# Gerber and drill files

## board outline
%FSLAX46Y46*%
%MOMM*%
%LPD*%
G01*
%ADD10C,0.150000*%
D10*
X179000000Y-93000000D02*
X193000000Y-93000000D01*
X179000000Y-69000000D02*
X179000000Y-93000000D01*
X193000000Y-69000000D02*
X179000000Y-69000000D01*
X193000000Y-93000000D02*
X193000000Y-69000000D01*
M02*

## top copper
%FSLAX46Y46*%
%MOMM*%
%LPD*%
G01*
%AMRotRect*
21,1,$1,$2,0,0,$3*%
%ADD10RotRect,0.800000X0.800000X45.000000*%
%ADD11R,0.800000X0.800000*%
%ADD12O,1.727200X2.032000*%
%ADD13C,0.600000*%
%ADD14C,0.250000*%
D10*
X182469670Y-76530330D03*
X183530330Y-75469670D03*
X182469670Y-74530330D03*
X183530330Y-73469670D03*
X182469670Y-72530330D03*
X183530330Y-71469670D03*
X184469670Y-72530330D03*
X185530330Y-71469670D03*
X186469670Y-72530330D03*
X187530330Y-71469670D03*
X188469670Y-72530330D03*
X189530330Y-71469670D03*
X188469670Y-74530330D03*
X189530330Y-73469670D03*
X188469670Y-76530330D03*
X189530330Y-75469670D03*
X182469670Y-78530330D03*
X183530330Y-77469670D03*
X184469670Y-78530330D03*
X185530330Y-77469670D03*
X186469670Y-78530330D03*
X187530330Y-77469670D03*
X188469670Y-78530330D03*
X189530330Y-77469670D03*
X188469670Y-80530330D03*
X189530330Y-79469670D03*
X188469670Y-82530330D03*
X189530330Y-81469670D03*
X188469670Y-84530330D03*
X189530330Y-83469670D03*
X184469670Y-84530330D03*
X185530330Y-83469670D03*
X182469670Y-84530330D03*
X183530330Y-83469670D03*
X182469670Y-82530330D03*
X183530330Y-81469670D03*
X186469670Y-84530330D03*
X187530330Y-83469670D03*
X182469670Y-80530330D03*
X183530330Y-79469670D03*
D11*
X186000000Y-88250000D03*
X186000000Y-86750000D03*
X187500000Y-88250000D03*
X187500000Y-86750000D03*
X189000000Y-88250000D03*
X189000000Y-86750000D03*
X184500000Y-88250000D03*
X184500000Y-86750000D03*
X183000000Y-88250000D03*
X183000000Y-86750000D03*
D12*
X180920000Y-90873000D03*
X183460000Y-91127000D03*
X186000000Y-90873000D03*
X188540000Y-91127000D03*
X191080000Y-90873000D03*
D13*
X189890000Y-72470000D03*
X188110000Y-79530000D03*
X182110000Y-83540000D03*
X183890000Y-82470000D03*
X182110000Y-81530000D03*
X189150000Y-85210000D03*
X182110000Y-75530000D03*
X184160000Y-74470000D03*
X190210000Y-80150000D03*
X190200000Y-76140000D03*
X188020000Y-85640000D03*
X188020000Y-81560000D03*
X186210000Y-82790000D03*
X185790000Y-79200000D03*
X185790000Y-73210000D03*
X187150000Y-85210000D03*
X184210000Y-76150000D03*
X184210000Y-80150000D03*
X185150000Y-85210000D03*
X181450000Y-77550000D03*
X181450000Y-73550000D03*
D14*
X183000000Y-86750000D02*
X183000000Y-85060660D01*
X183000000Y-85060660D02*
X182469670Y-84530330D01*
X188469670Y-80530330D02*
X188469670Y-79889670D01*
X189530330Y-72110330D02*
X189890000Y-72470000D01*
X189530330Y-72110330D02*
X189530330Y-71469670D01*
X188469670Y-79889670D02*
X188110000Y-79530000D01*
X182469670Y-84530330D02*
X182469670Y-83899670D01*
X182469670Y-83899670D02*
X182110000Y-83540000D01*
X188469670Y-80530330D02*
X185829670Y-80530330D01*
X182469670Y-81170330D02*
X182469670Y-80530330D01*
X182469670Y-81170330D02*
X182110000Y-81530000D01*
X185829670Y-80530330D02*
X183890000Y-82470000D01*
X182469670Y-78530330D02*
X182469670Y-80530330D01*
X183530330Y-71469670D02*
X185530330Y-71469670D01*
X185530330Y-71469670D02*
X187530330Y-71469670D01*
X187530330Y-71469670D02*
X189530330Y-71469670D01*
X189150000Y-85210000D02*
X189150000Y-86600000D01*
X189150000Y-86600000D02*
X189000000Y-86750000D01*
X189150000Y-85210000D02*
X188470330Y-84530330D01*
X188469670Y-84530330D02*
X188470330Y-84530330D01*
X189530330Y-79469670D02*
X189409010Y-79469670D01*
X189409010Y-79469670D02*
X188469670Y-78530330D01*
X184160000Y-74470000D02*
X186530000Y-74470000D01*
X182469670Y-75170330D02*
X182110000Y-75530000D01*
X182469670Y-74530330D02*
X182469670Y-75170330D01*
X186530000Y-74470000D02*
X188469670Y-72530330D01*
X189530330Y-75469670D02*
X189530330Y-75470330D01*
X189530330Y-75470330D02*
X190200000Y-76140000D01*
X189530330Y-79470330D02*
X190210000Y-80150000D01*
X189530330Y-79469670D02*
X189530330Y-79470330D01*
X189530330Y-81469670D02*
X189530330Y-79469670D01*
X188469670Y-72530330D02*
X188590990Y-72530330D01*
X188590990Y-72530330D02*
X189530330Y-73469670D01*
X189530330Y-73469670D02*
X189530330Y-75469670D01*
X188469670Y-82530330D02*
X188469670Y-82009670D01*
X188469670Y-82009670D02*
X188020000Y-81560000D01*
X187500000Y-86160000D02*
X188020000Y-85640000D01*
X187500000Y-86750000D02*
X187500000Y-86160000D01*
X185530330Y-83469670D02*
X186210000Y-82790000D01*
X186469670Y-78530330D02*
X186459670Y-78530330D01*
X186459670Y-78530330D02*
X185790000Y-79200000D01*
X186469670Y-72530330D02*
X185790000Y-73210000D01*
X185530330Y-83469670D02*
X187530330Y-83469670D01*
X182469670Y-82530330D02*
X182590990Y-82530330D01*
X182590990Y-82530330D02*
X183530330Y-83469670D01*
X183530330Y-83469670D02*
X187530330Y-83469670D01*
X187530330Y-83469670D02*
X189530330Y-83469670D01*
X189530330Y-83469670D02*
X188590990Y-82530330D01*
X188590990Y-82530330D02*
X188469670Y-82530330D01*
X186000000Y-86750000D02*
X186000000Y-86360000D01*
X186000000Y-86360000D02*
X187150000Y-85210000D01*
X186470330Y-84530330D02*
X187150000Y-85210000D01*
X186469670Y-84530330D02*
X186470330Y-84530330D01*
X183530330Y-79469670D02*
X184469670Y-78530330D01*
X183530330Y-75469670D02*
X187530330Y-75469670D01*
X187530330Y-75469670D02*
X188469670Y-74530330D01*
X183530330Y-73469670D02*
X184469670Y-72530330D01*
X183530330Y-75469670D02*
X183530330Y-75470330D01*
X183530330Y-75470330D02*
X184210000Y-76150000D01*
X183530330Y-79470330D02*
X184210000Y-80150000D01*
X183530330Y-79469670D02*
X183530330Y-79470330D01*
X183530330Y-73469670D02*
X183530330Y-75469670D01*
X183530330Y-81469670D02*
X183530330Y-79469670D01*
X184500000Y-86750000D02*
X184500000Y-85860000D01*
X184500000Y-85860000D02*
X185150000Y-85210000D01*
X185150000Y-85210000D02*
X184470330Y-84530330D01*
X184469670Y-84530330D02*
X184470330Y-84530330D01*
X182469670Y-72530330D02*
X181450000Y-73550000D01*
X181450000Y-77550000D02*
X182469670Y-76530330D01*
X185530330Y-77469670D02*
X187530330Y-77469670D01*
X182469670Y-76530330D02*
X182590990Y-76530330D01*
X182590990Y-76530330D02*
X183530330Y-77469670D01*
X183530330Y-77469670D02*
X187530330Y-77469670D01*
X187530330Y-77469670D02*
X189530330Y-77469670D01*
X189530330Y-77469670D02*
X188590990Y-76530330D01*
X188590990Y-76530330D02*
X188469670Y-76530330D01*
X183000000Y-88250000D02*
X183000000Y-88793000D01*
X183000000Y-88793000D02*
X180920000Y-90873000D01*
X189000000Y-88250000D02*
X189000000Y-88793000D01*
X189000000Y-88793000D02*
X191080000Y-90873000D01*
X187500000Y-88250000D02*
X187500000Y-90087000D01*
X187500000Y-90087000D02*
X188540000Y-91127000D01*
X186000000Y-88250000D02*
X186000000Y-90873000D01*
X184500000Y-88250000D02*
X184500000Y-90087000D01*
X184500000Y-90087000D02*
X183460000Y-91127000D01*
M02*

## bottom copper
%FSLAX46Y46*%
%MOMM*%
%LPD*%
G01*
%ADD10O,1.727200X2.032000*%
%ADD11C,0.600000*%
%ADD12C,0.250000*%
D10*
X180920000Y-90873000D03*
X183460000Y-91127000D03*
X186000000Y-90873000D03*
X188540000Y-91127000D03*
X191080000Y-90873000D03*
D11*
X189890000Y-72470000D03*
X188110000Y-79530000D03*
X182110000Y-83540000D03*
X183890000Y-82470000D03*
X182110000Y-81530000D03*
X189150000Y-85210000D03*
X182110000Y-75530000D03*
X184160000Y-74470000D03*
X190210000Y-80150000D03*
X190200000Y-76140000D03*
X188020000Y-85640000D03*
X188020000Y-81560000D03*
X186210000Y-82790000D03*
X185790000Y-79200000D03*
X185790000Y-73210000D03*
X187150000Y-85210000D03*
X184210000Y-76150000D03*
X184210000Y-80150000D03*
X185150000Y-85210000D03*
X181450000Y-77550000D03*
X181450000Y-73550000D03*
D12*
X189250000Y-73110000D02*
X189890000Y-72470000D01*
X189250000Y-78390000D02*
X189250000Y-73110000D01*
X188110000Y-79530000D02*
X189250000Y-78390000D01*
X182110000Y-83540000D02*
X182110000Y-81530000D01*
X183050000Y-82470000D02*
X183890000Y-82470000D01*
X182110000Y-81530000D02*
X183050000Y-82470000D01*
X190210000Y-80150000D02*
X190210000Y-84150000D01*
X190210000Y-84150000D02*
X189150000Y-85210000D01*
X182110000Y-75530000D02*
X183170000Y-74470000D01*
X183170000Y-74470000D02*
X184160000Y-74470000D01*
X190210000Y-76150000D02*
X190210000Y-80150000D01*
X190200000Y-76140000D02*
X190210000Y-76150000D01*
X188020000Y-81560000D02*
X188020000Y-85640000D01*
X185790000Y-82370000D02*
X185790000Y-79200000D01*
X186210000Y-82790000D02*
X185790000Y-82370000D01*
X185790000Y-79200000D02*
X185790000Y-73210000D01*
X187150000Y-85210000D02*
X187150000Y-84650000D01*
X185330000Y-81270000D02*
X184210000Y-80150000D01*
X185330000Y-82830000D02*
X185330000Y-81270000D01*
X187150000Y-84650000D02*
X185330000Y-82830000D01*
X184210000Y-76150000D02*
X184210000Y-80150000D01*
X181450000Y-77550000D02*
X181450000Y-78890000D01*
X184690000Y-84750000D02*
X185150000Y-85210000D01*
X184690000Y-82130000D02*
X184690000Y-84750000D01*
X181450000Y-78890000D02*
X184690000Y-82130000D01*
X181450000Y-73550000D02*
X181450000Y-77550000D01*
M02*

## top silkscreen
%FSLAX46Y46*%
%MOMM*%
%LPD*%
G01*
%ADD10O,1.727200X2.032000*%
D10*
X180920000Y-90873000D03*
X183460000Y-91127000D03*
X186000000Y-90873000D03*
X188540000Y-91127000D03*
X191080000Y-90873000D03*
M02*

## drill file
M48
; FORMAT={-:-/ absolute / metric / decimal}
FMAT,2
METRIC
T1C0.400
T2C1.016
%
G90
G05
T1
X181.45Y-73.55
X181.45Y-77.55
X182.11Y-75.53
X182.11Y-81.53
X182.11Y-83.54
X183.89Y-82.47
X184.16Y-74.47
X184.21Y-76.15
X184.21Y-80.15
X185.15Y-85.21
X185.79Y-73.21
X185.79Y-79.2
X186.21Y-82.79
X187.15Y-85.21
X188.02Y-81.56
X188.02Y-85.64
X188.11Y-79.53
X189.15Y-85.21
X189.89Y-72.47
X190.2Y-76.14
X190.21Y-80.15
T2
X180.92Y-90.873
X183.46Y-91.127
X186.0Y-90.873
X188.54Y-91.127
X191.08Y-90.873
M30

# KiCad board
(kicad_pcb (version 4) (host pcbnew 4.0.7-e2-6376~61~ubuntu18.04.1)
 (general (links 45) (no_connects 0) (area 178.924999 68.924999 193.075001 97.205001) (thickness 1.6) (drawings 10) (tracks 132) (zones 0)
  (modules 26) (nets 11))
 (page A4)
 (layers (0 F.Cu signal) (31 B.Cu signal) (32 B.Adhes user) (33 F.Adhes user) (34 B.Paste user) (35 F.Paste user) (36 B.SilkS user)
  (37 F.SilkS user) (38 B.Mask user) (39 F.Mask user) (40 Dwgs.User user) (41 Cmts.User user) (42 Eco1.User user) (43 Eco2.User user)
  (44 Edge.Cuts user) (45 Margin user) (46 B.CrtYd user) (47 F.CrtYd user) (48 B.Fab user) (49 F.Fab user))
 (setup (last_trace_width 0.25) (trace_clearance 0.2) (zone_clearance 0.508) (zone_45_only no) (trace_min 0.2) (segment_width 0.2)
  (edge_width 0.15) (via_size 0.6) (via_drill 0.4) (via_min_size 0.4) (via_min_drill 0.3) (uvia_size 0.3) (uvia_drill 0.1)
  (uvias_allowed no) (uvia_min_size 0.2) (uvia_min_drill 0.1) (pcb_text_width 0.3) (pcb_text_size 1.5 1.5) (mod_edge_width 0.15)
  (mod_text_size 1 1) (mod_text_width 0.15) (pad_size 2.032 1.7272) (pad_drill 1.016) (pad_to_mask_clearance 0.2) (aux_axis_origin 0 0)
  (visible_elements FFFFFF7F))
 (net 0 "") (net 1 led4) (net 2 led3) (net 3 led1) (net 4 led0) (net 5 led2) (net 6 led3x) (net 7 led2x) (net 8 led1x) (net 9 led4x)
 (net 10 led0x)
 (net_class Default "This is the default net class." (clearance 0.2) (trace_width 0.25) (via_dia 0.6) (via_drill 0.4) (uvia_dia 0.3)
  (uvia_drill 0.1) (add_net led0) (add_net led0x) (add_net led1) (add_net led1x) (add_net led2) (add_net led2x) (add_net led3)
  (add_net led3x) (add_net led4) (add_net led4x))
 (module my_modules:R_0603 (layer F.Cu) (at 183 76 45)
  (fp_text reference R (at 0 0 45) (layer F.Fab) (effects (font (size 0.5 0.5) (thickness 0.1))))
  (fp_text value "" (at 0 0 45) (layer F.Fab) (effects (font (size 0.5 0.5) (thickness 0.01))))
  (pad 1 smd rect (at -0.75 0 45) (size 0.8 0.8) (layers F.Cu F.Paste F.Mask) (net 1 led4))
  (pad 2 smd rect (at 0.75 0 45) (size 0.8 0.8) (layers F.Cu F.Paste F.Mask) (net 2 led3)))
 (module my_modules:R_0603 (layer F.Cu) (at 183 74 45)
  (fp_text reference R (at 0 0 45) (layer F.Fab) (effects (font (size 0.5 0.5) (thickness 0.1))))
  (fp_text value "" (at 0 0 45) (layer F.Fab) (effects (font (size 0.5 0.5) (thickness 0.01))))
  (pad 1 smd rect (at -0.75 0 45) (size 0.8 0.8) (layers F.Cu F.Paste F.Mask) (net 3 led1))
  (pad 2 smd rect (at 0.75 0 45) (size 0.8 0.8) (layers F.Cu F.Paste F.Mask) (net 2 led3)))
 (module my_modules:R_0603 (layer F.Cu) (at 183 72 45)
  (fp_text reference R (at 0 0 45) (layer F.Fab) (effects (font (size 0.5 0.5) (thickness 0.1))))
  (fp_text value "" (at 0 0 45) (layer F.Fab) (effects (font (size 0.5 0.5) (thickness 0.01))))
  (pad 1 smd rect (at -0.75 0 45) (size 0.8 0.8) (layers F.Cu F.Paste F.Mask) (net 1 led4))
  (pad 2 smd rect (at 0.75 0 45) (size 0.8 0.8) (layers F.Cu F.Paste F.Mask) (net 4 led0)))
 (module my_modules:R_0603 (layer F.Cu) (at 185 72 45)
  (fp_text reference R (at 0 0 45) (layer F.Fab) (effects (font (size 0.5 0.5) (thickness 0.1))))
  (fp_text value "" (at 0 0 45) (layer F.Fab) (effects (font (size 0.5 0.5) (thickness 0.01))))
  (pad 1 smd rect (at -0.75 0 45) (size 0.8 0.8) (layers F.Cu F.Paste F.Mask) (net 2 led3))
  (pad 2 smd rect (at 0.75 0 45) (size 0.8 0.8) (layers F.Cu F.Paste F.Mask) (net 4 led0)))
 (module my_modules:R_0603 (layer F.Cu) (at 187 72 45)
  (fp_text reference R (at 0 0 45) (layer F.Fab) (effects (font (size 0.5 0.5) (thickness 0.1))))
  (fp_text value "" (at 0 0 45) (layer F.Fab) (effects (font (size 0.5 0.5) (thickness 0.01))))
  (pad 1 smd rect (at -0.75 0 45) (size 0.8 0.8) (layers F.Cu F.Paste F.Mask) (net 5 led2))
  (pad 2 smd rect (at 0.75 0 45) (size 0.8 0.8) (layers F.Cu F.Paste F.Mask) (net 4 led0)))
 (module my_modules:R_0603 (layer F.Cu) (at 189 72 45)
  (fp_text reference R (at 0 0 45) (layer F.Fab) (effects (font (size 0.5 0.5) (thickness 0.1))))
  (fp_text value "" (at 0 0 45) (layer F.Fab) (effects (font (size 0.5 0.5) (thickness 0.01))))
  (pad 1 smd rect (at -0.75 0 45) (size 0.8 0.8) (layers F.Cu F.Paste F.Mask) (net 3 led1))
  (pad 2 smd rect (at 0.75 0 45) (size 0.8 0.8) (layers F.Cu F.Paste F.Mask) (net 4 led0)))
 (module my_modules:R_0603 (layer F.Cu) (at 189 74 45)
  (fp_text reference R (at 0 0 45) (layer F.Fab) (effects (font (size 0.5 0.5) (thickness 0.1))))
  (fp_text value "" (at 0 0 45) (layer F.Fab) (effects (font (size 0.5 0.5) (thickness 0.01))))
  (pad 1 smd rect (at -0.75 0 45) (size 0.8 0.8) (layers F.Cu F.Paste F.Mask) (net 2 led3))
  (pad 2 smd rect (at 0.75 0 45) (size 0.8 0.8) (layers F.Cu F.Paste F.Mask) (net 3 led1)))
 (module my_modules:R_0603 (layer F.Cu) (at 189 76 45)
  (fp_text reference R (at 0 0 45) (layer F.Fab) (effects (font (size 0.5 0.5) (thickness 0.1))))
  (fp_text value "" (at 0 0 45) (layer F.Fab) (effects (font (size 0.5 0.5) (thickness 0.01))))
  (pad 1 smd rect (at -0.75 0 45) (size 0.8 0.8) (layers F.Cu F.Paste F.Mask) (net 1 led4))
  (pad 2 smd rect (at 0.75 0 45) (size 0.8 0.8) (layers F.Cu F.Paste F.Mask) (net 3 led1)))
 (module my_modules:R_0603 (layer F.Cu) (at 183 78 45)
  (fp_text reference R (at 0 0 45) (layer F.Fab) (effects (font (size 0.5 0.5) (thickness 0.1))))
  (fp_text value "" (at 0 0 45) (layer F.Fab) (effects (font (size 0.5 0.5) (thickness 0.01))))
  (pad 1 smd rect (at -0.75 0 45) (size 0.8 0.8) (layers F.Cu F.Paste F.Mask) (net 4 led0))
  (pad 2 smd rect (at 0.75 0 45) (size 0.8 0.8) (layers F.Cu F.Paste F.Mask) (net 1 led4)))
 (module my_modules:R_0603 (layer F.Cu) (at 185 78 45)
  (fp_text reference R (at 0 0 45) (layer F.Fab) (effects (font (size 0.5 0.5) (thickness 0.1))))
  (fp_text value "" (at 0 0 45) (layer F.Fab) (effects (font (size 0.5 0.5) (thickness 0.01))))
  (pad 1 smd rect (at -0.75 0 45) (size 0.8 0.8) (layers F.Cu F.Paste F.Mask) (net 2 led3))
  (pad 2 smd rect (at 0.75 0 45) (size 0.8 0.8) (layers F.Cu F.Paste F.Mask) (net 1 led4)))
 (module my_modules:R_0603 (layer F.Cu) (at 187 78 45)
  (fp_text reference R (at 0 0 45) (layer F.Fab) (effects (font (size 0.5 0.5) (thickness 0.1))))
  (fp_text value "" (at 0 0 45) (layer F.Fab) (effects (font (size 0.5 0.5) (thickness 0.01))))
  (pad 1 smd rect (at -0.75 0 45) (size 0.8 0.8) (layers F.Cu F.Paste F.Mask) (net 5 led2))
  (pad 2 smd rect (at 0.75 0 45) (size 0.8 0.8) (layers F.Cu F.Paste F.Mask) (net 1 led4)))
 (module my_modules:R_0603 (layer F.Cu) (at 189 78 45)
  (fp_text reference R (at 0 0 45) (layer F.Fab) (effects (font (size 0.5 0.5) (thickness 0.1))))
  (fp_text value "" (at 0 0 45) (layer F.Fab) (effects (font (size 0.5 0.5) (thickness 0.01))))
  (pad 1 smd rect (at -0.75 0 45) (size 0.8 0.8) (layers F.Cu F.Paste F.Mask) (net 3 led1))
  (pad 2 smd rect (at 0.75 0 45) (size 0.8 0.8) (layers F.Cu F.Paste F.Mask) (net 1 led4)))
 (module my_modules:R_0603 (layer F.Cu) (at 189 80 45)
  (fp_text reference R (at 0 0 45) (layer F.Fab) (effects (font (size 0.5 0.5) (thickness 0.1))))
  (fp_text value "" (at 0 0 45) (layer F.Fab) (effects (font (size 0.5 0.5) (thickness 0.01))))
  (pad 1 smd rect (at -0.75 0 45) (size 0.8 0.8) (layers F.Cu F.Paste F.Mask) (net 4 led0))
  (pad 2 smd rect (at 0.75 0 45) (size 0.8 0.8) (layers F.Cu F.Paste F.Mask) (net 3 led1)))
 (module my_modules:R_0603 (layer F.Cu) (at 189 82 45)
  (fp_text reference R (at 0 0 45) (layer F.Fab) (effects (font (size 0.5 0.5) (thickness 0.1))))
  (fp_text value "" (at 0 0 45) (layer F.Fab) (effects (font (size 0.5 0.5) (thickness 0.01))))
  (pad 1 smd rect (at -0.75 0 45) (size 0.8 0.8) (layers F.Cu F.Paste F.Mask) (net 5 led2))
  (pad 2 smd rect (at 0.75 0 45) (size 0.8 0.8) (layers F.Cu F.Paste F.Mask) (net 3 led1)))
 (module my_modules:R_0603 (layer F.Cu) (at 189 84 45)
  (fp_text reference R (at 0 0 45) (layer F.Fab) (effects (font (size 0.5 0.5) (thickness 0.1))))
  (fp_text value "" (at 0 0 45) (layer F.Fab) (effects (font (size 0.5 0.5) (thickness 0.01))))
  (pad 1 smd rect (at -0.75 0 45) (size 0.8 0.8) (layers F.Cu F.Paste F.Mask) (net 3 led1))
  (pad 2 smd rect (at 0.75 0 45) (size 0.8 0.8) (layers F.Cu F.Paste F.Mask) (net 5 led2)))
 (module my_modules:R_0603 (layer F.Cu) (at 185 84 45)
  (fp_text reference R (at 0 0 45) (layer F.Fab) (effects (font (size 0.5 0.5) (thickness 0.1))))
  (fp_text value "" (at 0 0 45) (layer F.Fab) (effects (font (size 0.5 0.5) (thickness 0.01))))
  (pad 1 smd rect (at -0.75 0 45) (size 0.8 0.8) (layers F.Cu F.Paste F.Mask) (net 1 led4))
  (pad 2 smd rect (at 0.75 0 45) (size 0.8 0.8) (layers F.Cu F.Paste F.Mask) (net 5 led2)))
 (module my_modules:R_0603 (layer F.Cu) (at 183 84 45)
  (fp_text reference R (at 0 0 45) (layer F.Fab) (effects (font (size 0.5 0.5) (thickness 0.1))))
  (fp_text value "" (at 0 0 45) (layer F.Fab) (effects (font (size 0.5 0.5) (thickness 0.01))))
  (pad 1 smd rect (at -0.75 0 45) (size 0.8 0.8) (layers F.Cu F.Paste F.Mask) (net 4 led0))
  (pad 2 smd rect (at 0.75 0 45) (size 0.8 0.8) (layers F.Cu F.Paste F.Mask) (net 5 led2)))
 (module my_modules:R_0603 (layer F.Cu) (at 183 82 45)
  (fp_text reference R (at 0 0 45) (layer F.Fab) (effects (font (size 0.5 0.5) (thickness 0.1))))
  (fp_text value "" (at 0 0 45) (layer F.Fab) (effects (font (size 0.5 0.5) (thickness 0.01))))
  (pad 1 smd rect (at -0.75 0 45) (size 0.8 0.8) (layers F.Cu F.Paste F.Mask) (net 5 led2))
  (pad 2 smd rect (at 0.75 0 45) (size 0.8 0.8) (layers F.Cu F.Paste F.Mask) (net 2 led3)))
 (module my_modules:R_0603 (layer F.Cu) (at 187 84 45)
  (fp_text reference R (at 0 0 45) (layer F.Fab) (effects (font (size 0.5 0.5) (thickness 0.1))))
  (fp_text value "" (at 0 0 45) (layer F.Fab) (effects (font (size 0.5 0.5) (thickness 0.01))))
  (pad 1 smd rect (at -0.75 0 45) (size 0.8 0.8) (layers F.Cu F.Paste F.Mask) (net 2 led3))
  (pad 2 smd rect (at 0.75 0 45) (size 0.8 0.8) (layers F.Cu F.Paste F.Mask) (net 5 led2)))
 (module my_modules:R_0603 (layer F.Cu) (at 183 80 45)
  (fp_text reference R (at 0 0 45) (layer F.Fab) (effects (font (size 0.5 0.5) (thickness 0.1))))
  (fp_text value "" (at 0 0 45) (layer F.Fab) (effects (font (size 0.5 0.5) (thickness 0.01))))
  (pad 1 smd rect (at -0.75 0 45) (size 0.8 0.8) (layers F.Cu F.Paste F.Mask) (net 4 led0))
  (pad 2 smd rect (at 0.75 0 45) (size 0.8 0.8) (layers F.Cu F.Paste F.Mask) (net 2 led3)))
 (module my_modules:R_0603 (layer F.Cu) (at 186 87.5 90)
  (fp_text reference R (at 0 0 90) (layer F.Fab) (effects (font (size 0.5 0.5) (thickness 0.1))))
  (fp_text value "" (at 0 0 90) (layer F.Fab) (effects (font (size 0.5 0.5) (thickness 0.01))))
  (pad 1 smd rect (at -0.75 0 90) (size 0.8 0.8) (layers F.Cu F.Paste F.Mask) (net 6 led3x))
  (pad 2 smd rect (at 0.75 0 90) (size 0.8 0.8) (layers F.Cu F.Paste F.Mask) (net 2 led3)))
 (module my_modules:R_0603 (layer F.Cu) (at 187.5 87.5 90)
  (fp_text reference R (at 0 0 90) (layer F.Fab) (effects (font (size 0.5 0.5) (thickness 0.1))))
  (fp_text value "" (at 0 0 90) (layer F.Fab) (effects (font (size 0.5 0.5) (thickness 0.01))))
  (pad 1 smd rect (at -0.75 0 90) (size 0.8 0.8) (layers F.Cu F.Paste F.Mask) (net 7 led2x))
  (pad 2 smd rect (at 0.75 0 90) (size 0.8 0.8) (layers F.Cu F.Paste F.Mask) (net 5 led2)))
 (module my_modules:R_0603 (layer F.Cu) (at 189 87.5 90)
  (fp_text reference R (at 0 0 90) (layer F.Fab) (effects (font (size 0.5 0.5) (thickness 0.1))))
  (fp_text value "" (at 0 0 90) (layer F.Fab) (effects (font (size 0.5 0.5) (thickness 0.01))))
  (pad 1 smd rect (at -0.75 0 90) (size 0.8 0.8) (layers F.Cu F.Paste F.Mask) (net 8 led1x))
  (pad 2 smd rect (at 0.75 0 90) (size 0.8 0.8) (layers F.Cu F.Paste F.Mask) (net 3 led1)))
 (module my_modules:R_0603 (layer F.Cu) (at 184.5 87.5 90)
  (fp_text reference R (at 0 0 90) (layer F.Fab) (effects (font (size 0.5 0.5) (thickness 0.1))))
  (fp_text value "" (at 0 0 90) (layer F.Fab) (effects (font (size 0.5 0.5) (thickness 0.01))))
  (pad 1 smd rect (at -0.75 0 90) (size 0.8 0.8) (layers F.Cu F.Paste F.Mask) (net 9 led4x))
  (pad 2 smd rect (at 0.75 0 90) (size 0.8 0.8) (layers F.Cu F.Paste F.Mask) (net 1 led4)))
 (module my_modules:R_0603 (layer F.Cu) (at 183 87.5 90)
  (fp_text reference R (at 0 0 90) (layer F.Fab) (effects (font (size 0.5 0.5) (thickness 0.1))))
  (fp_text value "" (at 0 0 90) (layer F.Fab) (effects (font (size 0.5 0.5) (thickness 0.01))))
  (pad 1 smd rect (at -0.75 0 90) (size 0.8 0.8) (layers F.Cu F.Paste F.Mask) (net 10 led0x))
  (pad 2 smd rect (at 0.75 0 90) (size 0.8 0.8) (layers F.Cu F.Paste F.Mask) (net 4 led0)))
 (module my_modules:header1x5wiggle (layer F.Cu) (at 186 91 90)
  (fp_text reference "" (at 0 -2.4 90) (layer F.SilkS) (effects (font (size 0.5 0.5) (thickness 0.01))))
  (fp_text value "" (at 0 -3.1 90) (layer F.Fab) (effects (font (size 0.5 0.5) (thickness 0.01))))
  (pad 1 thru_hole oval (at 0.127 -5.08 90) (size 2.032 1.7272) (drill 1.016) (layers *.Cu *.Mask F.SilkS) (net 10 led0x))
  (pad 2 thru_hole oval (at -0.127 -2.54 90) (size 2.032 1.7272) (drill 1.016) (layers *.Cu *.Mask F.SilkS) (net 9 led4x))
  (pad 3 thru_hole oval (at 0.127 0 90) (size 2.032 1.7272) (drill 1.016) (layers *.Cu *.Mask F.SilkS) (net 6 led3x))
  (pad 4 thru_hole oval (at -0.127 2.54 90) (size 2.032 1.7272) (drill 1.016) (layers *.Cu *.Mask F.SilkS) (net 7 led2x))
  (pad 5 thru_hole oval (at 0.127 5.08 90) (size 2.032 1.7272) (drill 1.016) (layers *.Cu *.Mask F.SilkS) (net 8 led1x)))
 (gr_line (start 179 93) (end 193 93) (angle 90) (layer Edge.Cuts) (width 0.15))
 (gr_line (start 179 69) (end 179 93) (angle 90) (layer Edge.Cuts) (width 0.15))
 (gr_line (start 193 69) (end 179 69) (angle 90) (layer Edge.Cuts) (width 0.15))
 (gr_line (start 193 93) (end 193 69) (angle 90) (layer Edge.Cuts) (width 0.15))
 (segment (start 183 86.75) (end 183 85.06066) (width 0.25) (layer F.Cu) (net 4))
 (segment (start 183 85.06066) (end 182.46967 84.53033) (width 0.25) (layer F.Cu) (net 4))
 (segment (start 188.46967 80.53033) (end 188.46967 79.88967) (width 0.25) (layer F.Cu) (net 4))
 (segment (start 189.53033 72.11033) (end 189.89 72.47) (width 0.25) (layer F.Cu) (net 4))
 (via (at 189.89 72.47) (size 0.6) (drill 0.4) (layers F.Cu B.Cu) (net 4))
 (segment (start 189.53033 72.11033) (end 189.53033 71.46967) (width 0.25) (layer F.Cu) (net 4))
 (segment (start 189.25 73.11) (end 189.89 72.47) (width 0.25) (layer B.Cu) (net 4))
 (segment (start 189.25 78.39) (end 189.25 73.11) (width 0.25) (layer B.Cu) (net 4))
 (segment (start 188.11 79.53) (end 189.25 78.39) (width 0.25) (layer B.Cu) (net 4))
 (via (at 188.11 79.53) (size 0.6) (drill 0.4) (layers F.Cu B.Cu) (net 4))
 (segment (start 188.46967 79.88967) (end 188.11 79.53) (width 0.25) (layer F.Cu) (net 4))
 (segment (start 182.46967 84.53033) (end 182.46967 83.89967) (width 0.25) (layer F.Cu) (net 4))
 (segment (start 182.11 83.54) (end 182.11 81.53) (width 0.25) (layer B.Cu) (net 4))
 (via (at 182.11 83.54) (size 0.6) (drill 0.4) (layers F.Cu B.Cu) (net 4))
 (segment (start 182.46967 83.89967) (end 182.11 83.54) (width 0.25) (layer F.Cu) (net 4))
 (segment (start 188.46967 80.53033) (end 185.82967 80.53033) (width 0.25) (layer F.Cu) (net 4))
 (segment (start 182.46967 81.17033) (end 182.46967 80.53033) (width 0.25) (layer F.Cu) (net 4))
 (via (at 183.89 82.47) (size 0.6) (drill 0.4) (layers F.Cu B.Cu) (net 4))
 (segment (start 183.05 82.47) (end 183.89 82.47) (width 0.25) (layer B.Cu) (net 4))
 (segment (start 182.11 81.53) (end 183.05 82.47) (width 0.25) (layer B.Cu) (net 4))
 (via (at 182.11 81.53) (size 0.6) (drill 0.4) (layers F.Cu B.Cu) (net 4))
 (segment (start 182.46967 81.17033) (end 182.11 81.53) (width 0.25) (layer F.Cu) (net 4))
 (segment (start 185.82967 80.53033) (end 183.89 82.47) (width 0.25) (layer F.Cu) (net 4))
 (segment (start 182.46967 78.53033) (end 182.46967 80.53033) (width 0.25) (layer F.Cu) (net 4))
 (segment (start 183.53033 71.46967) (end 185.53033 71.46967) (width 0.25) (layer F.Cu) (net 4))
 (segment (start 185.53033 71.46967) (end 187.53033 71.46967) (width 0.25) (layer F.Cu) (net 4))
 (segment (start 187.53033 71.46967) (end 189.53033 71.46967) (width 0.25) (layer F.Cu) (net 4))
 (segment (start 189.15 85.21) (end 189.15 86.6) (width 0.25) (layer F.Cu) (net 3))
 (segment (start 189.15 86.6) (end 189 86.75) (width 0.25) (layer F.Cu) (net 3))
 (segment (start 190.21 80.15) (end 190.21 84.15) (width 0.25) (layer B.Cu) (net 3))
 (via (at 189.15 85.21) (size 0.6) (drill 0.4) (layers F.Cu B.Cu) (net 3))
 (segment (start 189.15 85.21) (end 188.47033 84.53033) (width 0.25) (layer F.Cu) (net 3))
 (segment (start 190.21 84.15) (end 189.15 85.21) (width 0.25) (layer B.Cu) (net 3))
 (segment (start 188.46967 84.53033) (end 188.47033 84.53033) (width 0.25) (layer F.Cu) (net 3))
 (segment (start 189.53033 79.46967) (end 189.40901 79.46967) (width 0.25) (layer F.Cu) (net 3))
 (segment (start 189.40901 79.46967) (end 188.46967 78.53033) (width 0.25) (layer F.Cu) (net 3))
 (segment (start 184.16 74.47) (end 186.53 74.47) (width 0.25) (layer F.Cu) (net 3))
 (segment (start 182.46967 75.17033) (end 182.11 75.53) (width 0.25) (layer F.Cu) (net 3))
 (via (at 182.11 75.53) (size 0.6) (drill 0.4) (layers F.Cu B.Cu) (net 3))
 (segment (start 182.11 75.53) (end 183.17 74.47) (width 0.25) (layer B.Cu) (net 3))
 (segment (start 183.17 74.47) (end 184.16 74.47) (width 0.25) (layer B.Cu) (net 3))
 (via (at 184.16 74.47) (size 0.6) (drill 0.4) (layers F.Cu B.Cu) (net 3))
 (segment (start 182.46967 74.53033) (end 182.46967 75.17033) (width 0.25) (layer F.Cu) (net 3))
 (segment (start 186.53 74.47) (end 188.46967 72.53033) (width 0.25) (layer F.Cu) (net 3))
 (segment (start 189.53033 75.46967) (end 189.53033 75.47033) (width 0.25) (layer F.Cu) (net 3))
 (segment (start 189.53033 75.47033) (end 190.2 76.14) (width 0.25) (layer F.Cu) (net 3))
 (via (at 190.21 80.15) (size 0.6) (drill 0.4) (layers F.Cu B.Cu) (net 3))
 (segment (start 189.53033 79.47033) (end 190.21 80.15) (width 0.25) (layer F.Cu) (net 3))
 (segment (start 190.21 76.15) (end 190.21 80.15) (width 0.25) (layer B.Cu) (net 3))
 (segment (start 190.2 76.14) (end 190.21 76.15) (width 0.25) (layer B.Cu) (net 3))
 (via (at 190.2 76.14) (size 0.6) (drill 0.4) (layers F.Cu B.Cu) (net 3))
 (segment (start 189.53033 79.46967) (end 189.53033 79.47033) (width 0.25) (layer F.Cu) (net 3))
 (segment (start 189.53033 81.46967) (end 189.53033 79.46967) (width 0.25) (layer F.Cu) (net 3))
 (segment (start 188.46967 72.53033) (end 188.59099 72.53033) (width 0.25) (layer F.Cu) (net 3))
 (segment (start 188.59099 72.53033) (end 189.53033 73.46967) (width 0.25) (layer F.Cu) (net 3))
 (segment (start 189.53033 73.46967) (end 189.53033 75.46967) (width 0.25) (layer F.Cu) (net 3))
 (segment (start 188.46967 82.53033) (end 188.46967 82.00967) (width 0.25) (layer F.Cu) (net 5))
 (segment (start 188.46967 82.00967) (end 188.02 81.56) (width 0.25) (layer F.Cu) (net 5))
 (segment (start 187.5 86.16) (end 188.02 85.64) (width 0.25) (layer F.Cu) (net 5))
 (via (at 188.02 85.64) (size 0.6) (drill 0.4) (layers F.Cu B.Cu) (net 5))
 (segment (start 187.5 86.75) (end 187.5 86.16) (width 0.25) (layer F.Cu) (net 5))
 (segment (start 188.02 81.56) (end 188.02 85.64) (width 0.25) (layer B.Cu) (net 5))
 (via (at 188.02 81.56) (size 0.6) (drill 0.4) (layers F.Cu B.Cu) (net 5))
 (segment (start 185.53033 83.46967) (end 186.21 82.79) (width 0.25) (layer F.Cu) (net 5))
 (segment (start 185.79 82.37) (end 185.79 79.2) (width 0.25) (layer B.Cu) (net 5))
 (segment (start 186.21 82.79) (end 185.79 82.37) (width 0.25) (layer B.Cu) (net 5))
 (via (at 186.21 82.79) (size 0.6) (drill 0.4) (layers F.Cu B.Cu) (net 5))
 (segment (start 186.46967 78.53033) (end 186.45967 78.53033) (width 0.25) (layer F.Cu) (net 5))
 (segment (start 186.45967 78.53033) (end 185.79 79.2) (width 0.25) (layer F.Cu) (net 5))
 (via (at 185.79 79.2) (size 0.6) (drill 0.4) (layers F.Cu B.Cu) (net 5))
 (segment (start 185.79 79.2) (end 185.79 73.21) (width 0.25) (layer B.Cu) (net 5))
 (via (at 185.79 73.21) (size 0.6) (drill 0.4) (layers F.Cu B.Cu) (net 5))
 (segment (start 186.46967 72.53033) (end 185.79 73.21) (width 0.25) (layer F.Cu) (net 5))
 (segment (start 185.53033 83.46967) (end 187.53033 83.46967) (width 0.25) (layer F.Cu) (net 5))
 (segment (start 182.46967 82.53033) (end 182.59099 82.53033) (width 0.25) (layer F.Cu) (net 5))
 (segment (start 182.59099 82.53033) (end 183.53033 83.46967) (width 0.25) (layer F.Cu) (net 5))
 (segment (start 183.53033 83.46967) (end 187.53033 83.46967) (width 0.25) (layer F.Cu) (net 5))
 (segment (start 187.53033 83.46967) (end 189.53033 83.46967) (width 0.25) (layer F.Cu) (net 5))
 (segment (start 189.53033 83.46967) (end 188.59099 82.53033) (width 0.25) (layer F.Cu) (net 5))
 (segment (start 188.59099 82.53033) (end 188.46967 82.53033) (width 0.25) (layer F.Cu) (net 5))
 (segment (start 186 86.75) (end 186 86.36) (width 0.25) (layer F.Cu) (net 2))
 (segment (start 186 86.36) (end 187.15 85.21) (width 0.25) (layer F.Cu) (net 2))
 (segment (start 187.15 85.21) (end 187.15 84.65) (width 0.25) (layer B.Cu) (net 2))
 (segment (start 186.47033 84.53033) (end 187.15 85.21) (width 0.25) (layer F.Cu) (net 2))
 (via (at 187.15 85.21) (size 0.6) (drill 0.4) (layers F.Cu B.Cu) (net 2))
 (segment (start 185.33 81.27) (end 184.21 80.15) (width 0.25) (layer B.Cu) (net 2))
 (segment (start 185.33 82.83) (end 185.33 81.27) (width 0.25) (layer B.Cu) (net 2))
 (segment (start 187.15 84.65) (end 185.33 82.83) (width 0.25) (layer B.Cu) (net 2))
 (segment (start 186.46967 84.53033) (end 186.47033 84.53033) (width 0.25) (layer F.Cu) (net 2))
 (segment (start 183.53033 79.46967) (end 184.46967 78.53033) (width 0.25) (layer F.Cu) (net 2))
 (segment (start 183.53033 75.46967) (end 187.53033 75.46967) (width 0.25) (layer F.Cu) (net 2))
 (segment (start 187.53033 75.46967) (end 188.46967 74.53033) (width 0.25) (layer F.Cu) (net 2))
 (segment (start 183.53033 73.46967) (end 184.46967 72.53033) (width 0.25) (layer F.Cu) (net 2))
 (segment (start 183.53033 75.46967) (end 183.53033 75.47033) (width 0.25) (layer F.Cu) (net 2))
 (segment (start 183.53033 75.47033) (end 184.21 76.15) (width 0.25) (layer F.Cu) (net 2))
 (segment (start 184.21 76.15) (end 184.21 80.15) (width 0.25) (layer B.Cu) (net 2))
 (via (at 184.21 76.15) (size 0.6) (drill 0.4) (layers F.Cu B.Cu) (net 2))
 (via (at 184.21 80.15) (size 0.6) (drill 0.4) (layers F.Cu B.Cu) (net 2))
 (segment (start 183.53033 79.47033) (end 184.21 80.15) (width 0.25) (layer F.Cu) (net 2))
 (segment (start 183.53033 79.46967) (end 183.53033 79.47033) (width 0.25) (layer F.Cu) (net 2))
 (segment (start 183.53033 73.46967) (end 183.53033 75.46967) (width 0.25) (layer F.Cu) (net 2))
 (segment (start 183.53033 81.46967) (end 183.53033 79.46967) (width 0.25) (layer F.Cu) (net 2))
 (segment (start 184.5 86.75) (end 184.5 85.86) (width 0.25) (layer F.Cu) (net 1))
 (segment (start 184.5 85.86) (end 185.15 85.21) (width 0.25) (layer F.Cu) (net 1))
 (segment (start 181.45 77.55) (end 181.45 78.89) (width 0.25) (layer B.Cu) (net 1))
 (via (at 185.15 85.21) (size 0.6) (drill 0.4) (layers F.Cu B.Cu) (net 1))
 (segment (start 185.15 85.21) (end 184.47033 84.53033) (width 0.25) (layer F.Cu) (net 1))
 (segment (start 184.69 84.75) (end 185.15 85.21) (width 0.25) (layer B.Cu) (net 1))
 (segment (start 184.69 82.13) (end 184.69 84.75) (width 0.25) (layer B.Cu) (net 1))
 (segment (start 181.45 78.89) (end 184.69 82.13) (width 0.25) (layer B.Cu) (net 1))
 (segment (start 184.46967 84.53033) (end 184.47033 84.53033) (width 0.25) (layer F.Cu) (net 1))
 (segment (start 182.46967 72.53033) (end 181.45 73.55) (width 0.25) (layer F.Cu) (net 1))
 (via (at 181.45 77.55) (size 0.6) (drill 0.4) (layers F.Cu B.Cu) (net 1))
 (segment (start 181.45 77.55) (end 182.46967 76.53033) (width 0.25) (layer F.Cu) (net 1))
 (segment (start 181.45 73.55) (end 181.45 77.55) (width 0.25) (layer B.Cu) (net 1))
 (via (at 181.45 73.55) (size 0.6) (drill 0.4) (layers F.Cu B.Cu) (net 1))
 (segment (start 185.53033 77.46967) (end 187.53033 77.46967) (width 0.25) (layer F.Cu) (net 1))
 (segment (start 182.46967 76.53033) (end 182.59099 76.53033) (width 0.25) (layer F.Cu) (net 1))
 (segment (start 182.59099 76.53033) (end 183.53033 77.46967) (width 0.25) (layer F.Cu) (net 1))
 (segment (start 183.53033 77.46967) (end 187.53033 77.46967) (width 0.25) (layer F.Cu) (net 1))
 (segment (start 187.53033 77.46967) (end 189.53033 77.46967) (width 0.25) (layer F.Cu) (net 1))
 (segment (start 189.53033 77.46967) (end 188.59099 76.53033) (width 0.25) (layer F.Cu) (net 1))
 (segment (start 188.59099 76.53033) (end 188.46967 76.53033) (width 0.25) (layer F.Cu) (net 1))
 (segment (start 183 88.25) (end 183 88.793) (width 0.25) (layer F.Cu) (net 10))
 (segment (start 183 88.793) (end 180.92 90.873) (width 0.25) (layer F.Cu) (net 10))
 (segment (start 189 88.25) (end 189 88.793) (width 0.25) (layer F.Cu) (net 8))
 (segment (start 189 88.793) (end 191.08 90.873) (width 0.25) (layer F.Cu) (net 8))
 (segment (start 187.5 88.25) (end 187.5 90.087) (width 0.25) (layer F.Cu) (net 7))
 (segment (start 187.5 90.087) (end 188.54 91.127) (width 0.25) (layer F.Cu) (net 7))
 (segment (start 186 88.25) (end 186 90.873) (width 0.25) (layer F.Cu) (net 6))
 (segment (start 184.5 88.25) (end 184.5 90.087) (width 0.25) (layer F.Cu) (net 9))
 (segment (start 184.5 90.087) (end 183.46 91.127) (width 0.25) (layer F.Cu) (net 9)))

